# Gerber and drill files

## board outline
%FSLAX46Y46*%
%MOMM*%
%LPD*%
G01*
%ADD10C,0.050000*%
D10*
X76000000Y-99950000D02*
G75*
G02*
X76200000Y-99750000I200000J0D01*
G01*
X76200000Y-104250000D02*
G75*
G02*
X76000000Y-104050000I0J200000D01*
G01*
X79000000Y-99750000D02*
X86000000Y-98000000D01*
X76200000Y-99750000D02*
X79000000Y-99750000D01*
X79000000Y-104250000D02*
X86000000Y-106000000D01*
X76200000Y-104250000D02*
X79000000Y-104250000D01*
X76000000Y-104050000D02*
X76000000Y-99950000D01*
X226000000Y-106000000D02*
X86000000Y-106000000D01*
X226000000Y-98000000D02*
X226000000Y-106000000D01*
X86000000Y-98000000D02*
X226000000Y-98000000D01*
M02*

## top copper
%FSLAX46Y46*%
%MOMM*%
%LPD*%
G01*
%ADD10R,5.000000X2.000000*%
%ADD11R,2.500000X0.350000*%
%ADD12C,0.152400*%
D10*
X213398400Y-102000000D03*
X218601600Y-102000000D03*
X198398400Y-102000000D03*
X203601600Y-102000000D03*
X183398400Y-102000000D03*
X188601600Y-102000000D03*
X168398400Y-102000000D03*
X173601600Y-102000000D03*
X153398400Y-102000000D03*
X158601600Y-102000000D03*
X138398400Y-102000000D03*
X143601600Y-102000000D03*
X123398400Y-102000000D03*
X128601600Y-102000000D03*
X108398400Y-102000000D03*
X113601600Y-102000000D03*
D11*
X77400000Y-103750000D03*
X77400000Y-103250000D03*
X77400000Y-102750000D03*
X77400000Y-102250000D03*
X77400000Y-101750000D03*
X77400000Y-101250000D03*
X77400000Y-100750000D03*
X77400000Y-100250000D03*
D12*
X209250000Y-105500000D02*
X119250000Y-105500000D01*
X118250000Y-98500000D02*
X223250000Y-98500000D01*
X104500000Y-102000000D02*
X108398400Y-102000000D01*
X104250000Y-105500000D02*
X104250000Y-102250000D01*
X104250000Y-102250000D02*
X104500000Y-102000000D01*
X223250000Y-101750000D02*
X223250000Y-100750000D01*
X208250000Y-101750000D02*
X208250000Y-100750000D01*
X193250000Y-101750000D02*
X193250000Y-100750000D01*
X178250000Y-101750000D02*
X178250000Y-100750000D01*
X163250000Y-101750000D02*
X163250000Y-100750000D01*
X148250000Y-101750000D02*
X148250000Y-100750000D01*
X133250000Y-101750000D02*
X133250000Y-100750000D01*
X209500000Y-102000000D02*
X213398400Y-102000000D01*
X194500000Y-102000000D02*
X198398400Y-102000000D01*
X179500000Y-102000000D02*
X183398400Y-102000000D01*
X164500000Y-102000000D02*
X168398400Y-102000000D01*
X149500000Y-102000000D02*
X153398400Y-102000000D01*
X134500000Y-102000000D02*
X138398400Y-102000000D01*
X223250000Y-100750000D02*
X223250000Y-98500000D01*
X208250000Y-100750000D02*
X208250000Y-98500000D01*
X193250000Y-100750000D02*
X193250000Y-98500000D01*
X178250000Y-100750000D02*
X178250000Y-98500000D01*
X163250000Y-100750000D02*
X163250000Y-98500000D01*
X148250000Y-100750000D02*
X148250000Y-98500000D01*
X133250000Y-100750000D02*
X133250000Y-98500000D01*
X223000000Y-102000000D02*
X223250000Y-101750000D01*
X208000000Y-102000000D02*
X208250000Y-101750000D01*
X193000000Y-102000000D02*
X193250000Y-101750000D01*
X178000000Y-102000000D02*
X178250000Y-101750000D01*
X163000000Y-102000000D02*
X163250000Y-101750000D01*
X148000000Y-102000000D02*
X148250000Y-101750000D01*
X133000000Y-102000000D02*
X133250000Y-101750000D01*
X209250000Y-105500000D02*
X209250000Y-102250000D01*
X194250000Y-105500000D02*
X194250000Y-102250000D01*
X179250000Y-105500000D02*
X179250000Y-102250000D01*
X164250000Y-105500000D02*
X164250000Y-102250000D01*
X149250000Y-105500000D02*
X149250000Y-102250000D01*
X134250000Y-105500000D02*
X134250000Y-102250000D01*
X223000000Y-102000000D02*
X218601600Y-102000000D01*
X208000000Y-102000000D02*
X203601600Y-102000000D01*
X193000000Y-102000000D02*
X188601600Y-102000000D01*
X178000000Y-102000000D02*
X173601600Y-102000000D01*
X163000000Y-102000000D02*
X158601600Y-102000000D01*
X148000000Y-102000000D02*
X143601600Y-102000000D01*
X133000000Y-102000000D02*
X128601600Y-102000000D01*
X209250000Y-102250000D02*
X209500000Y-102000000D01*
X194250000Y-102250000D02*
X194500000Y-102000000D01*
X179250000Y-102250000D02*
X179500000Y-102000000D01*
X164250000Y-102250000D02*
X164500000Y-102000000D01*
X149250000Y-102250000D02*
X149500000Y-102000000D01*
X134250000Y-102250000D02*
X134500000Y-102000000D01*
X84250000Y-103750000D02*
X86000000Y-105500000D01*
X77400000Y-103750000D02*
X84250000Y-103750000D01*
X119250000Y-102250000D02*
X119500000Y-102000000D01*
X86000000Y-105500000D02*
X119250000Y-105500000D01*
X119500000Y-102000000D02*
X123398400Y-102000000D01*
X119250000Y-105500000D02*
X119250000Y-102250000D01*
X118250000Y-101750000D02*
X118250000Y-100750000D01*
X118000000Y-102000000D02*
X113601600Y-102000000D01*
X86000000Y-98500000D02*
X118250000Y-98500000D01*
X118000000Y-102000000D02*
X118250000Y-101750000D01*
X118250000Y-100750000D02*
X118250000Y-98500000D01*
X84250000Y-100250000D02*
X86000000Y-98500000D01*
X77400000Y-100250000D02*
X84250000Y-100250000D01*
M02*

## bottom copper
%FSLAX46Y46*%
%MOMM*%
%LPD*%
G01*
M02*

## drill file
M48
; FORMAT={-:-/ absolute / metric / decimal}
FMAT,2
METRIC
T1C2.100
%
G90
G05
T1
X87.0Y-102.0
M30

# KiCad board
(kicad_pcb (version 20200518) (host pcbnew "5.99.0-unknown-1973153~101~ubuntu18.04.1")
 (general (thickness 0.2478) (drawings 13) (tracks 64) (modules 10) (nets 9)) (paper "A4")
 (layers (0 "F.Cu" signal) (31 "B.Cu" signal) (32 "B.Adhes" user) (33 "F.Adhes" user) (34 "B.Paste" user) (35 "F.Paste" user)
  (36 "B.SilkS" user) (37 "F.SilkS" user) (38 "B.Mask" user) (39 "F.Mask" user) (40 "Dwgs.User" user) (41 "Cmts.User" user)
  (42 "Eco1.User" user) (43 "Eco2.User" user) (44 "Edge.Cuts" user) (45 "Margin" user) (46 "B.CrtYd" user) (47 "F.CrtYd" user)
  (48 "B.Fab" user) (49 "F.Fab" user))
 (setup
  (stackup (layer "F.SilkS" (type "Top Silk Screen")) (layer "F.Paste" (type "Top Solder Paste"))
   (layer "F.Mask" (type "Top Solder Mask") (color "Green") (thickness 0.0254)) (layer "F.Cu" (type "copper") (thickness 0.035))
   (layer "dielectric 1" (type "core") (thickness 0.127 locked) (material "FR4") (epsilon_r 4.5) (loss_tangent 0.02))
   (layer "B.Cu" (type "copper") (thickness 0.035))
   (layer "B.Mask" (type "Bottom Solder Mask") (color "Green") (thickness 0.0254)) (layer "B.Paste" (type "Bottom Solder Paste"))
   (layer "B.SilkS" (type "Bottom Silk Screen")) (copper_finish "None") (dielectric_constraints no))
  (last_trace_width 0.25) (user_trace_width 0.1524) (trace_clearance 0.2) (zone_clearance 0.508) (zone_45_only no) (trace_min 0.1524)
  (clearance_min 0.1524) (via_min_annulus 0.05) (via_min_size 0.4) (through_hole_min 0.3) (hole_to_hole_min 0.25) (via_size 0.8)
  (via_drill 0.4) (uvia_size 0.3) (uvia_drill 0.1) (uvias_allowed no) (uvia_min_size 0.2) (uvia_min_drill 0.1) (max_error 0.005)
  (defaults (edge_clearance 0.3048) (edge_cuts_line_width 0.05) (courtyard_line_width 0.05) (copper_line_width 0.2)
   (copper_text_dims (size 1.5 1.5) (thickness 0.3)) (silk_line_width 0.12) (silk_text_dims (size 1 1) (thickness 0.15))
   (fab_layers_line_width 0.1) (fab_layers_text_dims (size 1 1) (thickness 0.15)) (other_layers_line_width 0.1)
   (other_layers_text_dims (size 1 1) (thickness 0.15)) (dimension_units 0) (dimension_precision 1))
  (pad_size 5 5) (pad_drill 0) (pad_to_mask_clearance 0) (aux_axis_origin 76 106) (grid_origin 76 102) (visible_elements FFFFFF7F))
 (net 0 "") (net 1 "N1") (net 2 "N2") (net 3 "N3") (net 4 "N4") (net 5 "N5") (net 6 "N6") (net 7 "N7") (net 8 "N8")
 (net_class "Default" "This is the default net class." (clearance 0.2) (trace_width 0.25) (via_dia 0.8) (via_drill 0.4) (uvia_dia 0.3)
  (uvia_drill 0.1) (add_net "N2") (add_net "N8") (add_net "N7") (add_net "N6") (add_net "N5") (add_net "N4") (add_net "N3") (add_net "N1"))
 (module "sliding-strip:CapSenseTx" (layer "F.Cu") (at 216 102)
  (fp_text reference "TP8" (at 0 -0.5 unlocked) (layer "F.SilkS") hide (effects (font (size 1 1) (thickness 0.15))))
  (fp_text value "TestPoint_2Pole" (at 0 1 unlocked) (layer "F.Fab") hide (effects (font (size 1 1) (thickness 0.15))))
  (pad "1" smd rect (at -2.6016 0) (size 5 2) (layers "F.Cu") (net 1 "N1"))
  (pad "2" smd rect (at 2.6016 0) (size 5 2) (layers "F.Cu") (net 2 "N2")))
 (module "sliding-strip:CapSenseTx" (layer "F.Cu") (at 201 102)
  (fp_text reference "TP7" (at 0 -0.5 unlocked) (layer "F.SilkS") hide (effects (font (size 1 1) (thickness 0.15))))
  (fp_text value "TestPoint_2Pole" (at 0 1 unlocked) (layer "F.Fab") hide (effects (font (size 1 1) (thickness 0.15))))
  (pad "1" smd rect (at -2.6016 0) (size 5 2) (layers "F.Cu") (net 1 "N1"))
  (pad "2" smd rect (at 2.6016 0) (size 5 2) (layers "F.Cu") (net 2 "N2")))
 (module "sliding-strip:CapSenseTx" (layer "F.Cu") (at 186 102)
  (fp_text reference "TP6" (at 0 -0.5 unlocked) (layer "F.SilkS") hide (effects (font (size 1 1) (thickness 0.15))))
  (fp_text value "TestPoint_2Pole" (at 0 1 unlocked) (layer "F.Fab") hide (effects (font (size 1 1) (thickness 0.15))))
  (pad "1" smd rect (at -2.6016 0) (size 5 2) (layers "F.Cu") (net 1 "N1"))
  (pad "2" smd rect (at 2.6016 0) (size 5 2) (layers "F.Cu") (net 2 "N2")))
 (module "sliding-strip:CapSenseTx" (layer "F.Cu") (at 171 102)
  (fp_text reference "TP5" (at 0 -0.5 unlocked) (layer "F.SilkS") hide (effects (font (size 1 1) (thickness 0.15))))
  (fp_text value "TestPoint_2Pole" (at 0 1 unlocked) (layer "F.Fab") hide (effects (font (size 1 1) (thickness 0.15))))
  (pad "1" smd rect (at -2.6016 0) (size 5 2) (layers "F.Cu") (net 1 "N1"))
  (pad "2" smd rect (at 2.6016 0) (size 5 2) (layers "F.Cu") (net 2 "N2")))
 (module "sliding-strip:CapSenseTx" (layer "F.Cu") (at 156 102)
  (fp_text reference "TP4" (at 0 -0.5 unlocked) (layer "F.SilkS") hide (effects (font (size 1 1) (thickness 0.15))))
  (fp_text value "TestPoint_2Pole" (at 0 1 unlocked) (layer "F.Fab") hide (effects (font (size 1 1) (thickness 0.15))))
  (pad "1" smd rect (at -2.6016 0) (size 5 2) (layers "F.Cu") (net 1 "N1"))
  (pad "2" smd rect (at 2.6016 0) (size 5 2) (layers "F.Cu") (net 2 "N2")))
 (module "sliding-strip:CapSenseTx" (layer "F.Cu") (at 141 102)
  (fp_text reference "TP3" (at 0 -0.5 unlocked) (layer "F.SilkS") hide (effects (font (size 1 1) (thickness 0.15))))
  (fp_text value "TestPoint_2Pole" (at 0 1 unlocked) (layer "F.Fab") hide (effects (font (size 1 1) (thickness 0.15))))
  (pad "1" smd rect (at -2.6016 0) (size 5 2) (layers "F.Cu") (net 1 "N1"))
  (pad "2" smd rect (at 2.6016 0) (size 5 2) (layers "F.Cu") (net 2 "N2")))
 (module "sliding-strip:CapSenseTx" (layer "F.Cu") (at 126 102)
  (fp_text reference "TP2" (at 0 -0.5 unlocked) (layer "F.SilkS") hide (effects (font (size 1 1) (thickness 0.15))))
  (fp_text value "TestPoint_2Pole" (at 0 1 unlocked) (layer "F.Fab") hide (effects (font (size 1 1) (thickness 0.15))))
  (pad "1" smd rect (at -2.6016 0) (size 5 2) (layers "F.Cu") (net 1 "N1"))
  (pad "2" smd rect (at 2.6016 0) (size 5 2) (layers "F.Cu") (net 2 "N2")))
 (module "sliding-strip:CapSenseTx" (layer "F.Cu") (at 111 102)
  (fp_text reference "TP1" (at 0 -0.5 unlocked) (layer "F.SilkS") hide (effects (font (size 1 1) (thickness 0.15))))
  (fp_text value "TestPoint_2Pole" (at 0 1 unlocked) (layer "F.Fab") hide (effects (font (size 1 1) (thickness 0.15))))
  (pad "1" smd rect (at -2.6016 0) (size 5 2) (layers "F.Cu") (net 1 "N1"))
  (pad "2" smd rect (at 2.6016 0) (size 5 2) (layers "F.Cu") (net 2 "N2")))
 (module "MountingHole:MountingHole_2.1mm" (layer "F.Cu") (at 87 102)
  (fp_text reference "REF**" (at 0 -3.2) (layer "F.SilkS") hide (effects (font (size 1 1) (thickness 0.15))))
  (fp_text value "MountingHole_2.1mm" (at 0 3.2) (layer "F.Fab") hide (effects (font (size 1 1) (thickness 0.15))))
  (pad "" np_thru_hole circle (at 0 0) (size 2.1 2.1) (drill 2.1) (layers *.Cu *.Mask)))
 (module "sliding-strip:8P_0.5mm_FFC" (layer "F.Cu") (at 77.4 102 -90)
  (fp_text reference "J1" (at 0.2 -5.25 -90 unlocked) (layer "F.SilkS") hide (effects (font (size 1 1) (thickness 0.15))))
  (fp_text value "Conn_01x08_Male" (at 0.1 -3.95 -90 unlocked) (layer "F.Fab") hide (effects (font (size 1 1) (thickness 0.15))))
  (pad "8" smd rect (at 1.75 0 270) (size 0.35 2.5) (layers "F.Cu" "F.Mask") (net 1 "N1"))
  (pad "7" smd rect (at 1.25 0 270) (size 0.35 2.5) (layers "F.Cu" "F.Mask") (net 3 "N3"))
  (pad "6" smd rect (at 0.75 0 270) (size 0.35 2.5) (layers "F.Cu" "F.Mask") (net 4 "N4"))
  (pad "5" smd rect (at 0.25 0 270) (size 0.35 2.5) (layers "F.Cu" "F.Mask") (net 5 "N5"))
  (pad "4" smd rect (at -0.25 0 270) (size 0.35 2.5) (layers "F.Cu" "F.Mask") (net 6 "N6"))
  (pad "3" smd rect (at -0.75 0 270) (size 0.35 2.5) (layers "F.Cu" "F.Mask") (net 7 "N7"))
  (pad "2" smd rect (at -1.25 0 270) (size 0.35 2.5) (layers "F.Cu" "F.Mask") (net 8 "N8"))
  (pad "1" smd rect (at -1.75 0 270) (size 0.35 2.5) (layers "F.Cu" "F.Mask") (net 2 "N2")))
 (gr_arc (start 76.2 99.95) (end 76.2 99.75) (angle -90) (layer "Edge.Cuts") (width 0.05))
 (gr_arc (start 76.2 104.05) (end 76 104.05) (angle -90) (layer "Edge.Cuts") (width 0.05))
 (gr_line (start 79 99.75) (end 86 98) (layer "Edge.Cuts") (width 0.05))
 (gr_line (start 76.2 99.75) (end 79 99.75) (layer "Edge.Cuts") (width 0.05))
 (gr_line (start 79 104.25) (end 86 106) (layer "Edge.Cuts") (width 0.05))
 (gr_line (start 76.2 104.25) (end 79 104.25) (layer "Edge.Cuts") (width 0.05))
 (gr_line (start 76 104.05) (end 76 99.95) (layer "Edge.Cuts") (width 0.05))
 (gr_line (start 226 106) (end 86 106) (layer "Edge.Cuts") (width 0.05))
 (gr_line (start 226 98) (end 226 106) (layer "Edge.Cuts") (width 0.05))
 (gr_line (start 86 98) (end 226 98) (layer "Edge.Cuts") (width 0.05))
 (segment (start 209.25 105.5) (end 119.25 105.5) (width 0.1524) (layer "F.Cu") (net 1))
 (segment (start 118.25 98.5) (end 223.25 98.5) (width 0.1524) (layer "F.Cu") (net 2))
 (segment (start 104.5 102) (end 108.3984 102) (width 0.1524) (layer "F.Cu") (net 1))
 (segment (start 104.25 105.5) (end 104.25 102.25) (width 0.1524) (layer "F.Cu") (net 1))
 (segment (start 104.25 102.25) (end 104.5 102) (width 0.1524) (layer "F.Cu") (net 1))
 (segment (start 223.25 101.75) (end 223.25 100.75) (width 0.1524) (layer "F.Cu") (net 2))
 (segment (start 208.25 101.75) (end 208.25 100.75) (width 0.1524) (layer "F.Cu") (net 2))
 (segment (start 193.25 101.75) (end 193.25 100.75) (width 0.1524) (layer "F.Cu") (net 2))
 (segment (start 178.25 101.75) (end 178.25 100.75) (width 0.1524) (layer "F.Cu") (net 2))
 (segment (start 163.25 101.75) (end 163.25 100.75) (width 0.1524) (layer "F.Cu") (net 2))
 (segment (start 148.25 101.75) (end 148.25 100.75) (width 0.1524) (layer "F.Cu") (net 2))
 (segment (start 133.25 101.75) (end 133.25 100.75) (width 0.1524) (layer "F.Cu") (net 2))
 (segment (start 209.5 102) (end 213.3984 102) (width 0.1524) (layer "F.Cu") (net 1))
 (segment (start 194.5 102) (end 198.3984 102) (width 0.1524) (layer "F.Cu") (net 1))
 (segment (start 179.5 102) (end 183.3984 102) (width 0.1524) (layer "F.Cu") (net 1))
 (segment (start 164.5 102) (end 168.3984 102) (width 0.1524) (layer "F.Cu") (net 1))
 (segment (start 149.5 102) (end 153.3984 102) (width 0.1524) (layer "F.Cu") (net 1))
 (segment (start 134.5 102) (end 138.3984 102) (width 0.1524) (layer "F.Cu") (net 1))
 (segment (start 223.25 100.75) (end 223.25 98.5) (width 0.1524) (layer "F.Cu") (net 2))
 (segment (start 208.25 100.75) (end 208.25 98.5) (width 0.1524) (layer "F.Cu") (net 2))
 (segment (start 193.25 100.75) (end 193.25 98.5) (width 0.1524) (layer "F.Cu") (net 2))
 (segment (start 178.25 100.75) (end 178.25 98.5) (width 0.1524) (layer "F.Cu") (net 2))
 (segment (start 163.25 100.75) (end 163.25 98.5) (width 0.1524) (layer "F.Cu") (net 2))
 (segment (start 148.25 100.75) (end 148.25 98.5) (width 0.1524) (layer "F.Cu") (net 2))
 (segment (start 133.25 100.75) (end 133.25 98.5) (width 0.1524) (layer "F.Cu") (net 2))
 (segment (start 223 102) (end 223.25 101.75) (width 0.1524) (layer "F.Cu") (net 2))
 (segment (start 208 102) (end 208.25 101.75) (width 0.1524) (layer "F.Cu") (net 2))
 (segment (start 193 102) (end 193.25 101.75) (width 0.1524) (layer "F.Cu") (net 2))
 (segment (start 178 102) (end 178.25 101.75) (width 0.1524) (layer "F.Cu") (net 2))
 (segment (start 163 102) (end 163.25 101.75) (width 0.1524) (layer "F.Cu") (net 2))
 (segment (start 148 102) (end 148.25 101.75) (width 0.1524) (layer "F.Cu") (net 2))
 (segment (start 133 102) (end 133.25 101.75) (width 0.1524) (layer "F.Cu") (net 2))
 (segment (start 209.25 105.5) (end 209.25 102.25) (width 0.1524) (layer "F.Cu") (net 1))
 (segment (start 194.25 105.5) (end 194.25 102.25) (width 0.1524) (layer "F.Cu") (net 1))
 (segment (start 179.25 105.5) (end 179.25 102.25) (width 0.1524) (layer "F.Cu") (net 1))
 (segment (start 164.25 105.5) (end 164.25 102.25) (width 0.1524) (layer "F.Cu") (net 1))
 (segment (start 149.25 105.5) (end 149.25 102.25) (width 0.1524) (layer "F.Cu") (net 1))
 (segment (start 134.25 105.5) (end 134.25 102.25) (width 0.1524) (layer "F.Cu") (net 1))
 (segment (start 223 102) (end 218.6016 102) (width 0.1524) (layer "F.Cu") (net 2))
 (segment (start 208 102) (end 203.6016 102) (width 0.1524) (layer "F.Cu") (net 2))
 (segment (start 193 102) (end 188.6016 102) (width 0.1524) (layer "F.Cu") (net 2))
 (segment (start 178 102) (end 173.6016 102) (width 0.1524) (layer "F.Cu") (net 2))
 (segment (start 163 102) (end 158.6016 102) (width 0.1524) (layer "F.Cu") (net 2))
 (segment (start 148 102) (end 143.6016 102) (width 0.1524) (layer "F.Cu") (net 2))
 (segment (start 133 102) (end 128.6016 102) (width 0.1524) (layer "F.Cu") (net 2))
 (segment (start 209.25 102.25) (end 209.5 102) (width 0.1524) (layer "F.Cu") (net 1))
 (segment (start 194.25 102.25) (end 194.5 102) (width 0.1524) (layer "F.Cu") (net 1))
 (segment (start 179.25 102.25) (end 179.5 102) (width 0.1524) (layer "F.Cu") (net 1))
 (segment (start 164.25 102.25) (end 164.5 102) (width 0.1524) (layer "F.Cu") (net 1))
 (segment (start 149.25 102.25) (end 149.5 102) (width 0.1524) (layer "F.Cu") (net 1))
 (segment (start 134.25 102.25) (end 134.5 102) (width 0.1524) (layer "F.Cu") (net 1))
 (segment (start 84.25 103.75) (end 86 105.5) (width 0.1524) (layer "F.Cu") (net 1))
 (segment (start 77.4 103.75) (end 84.25 103.75) (width 0.1524) (layer "F.Cu") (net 1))
 (segment (start 119.25 102.25) (end 119.5 102) (width 0.1524) (layer "F.Cu") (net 1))
 (segment (start 86 105.5) (end 119.25 105.5) (width 0.1524) (layer "F.Cu") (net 1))
 (segment (start 119.5 102) (end 123.3984 102) (width 0.1524) (layer "F.Cu") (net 1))
 (segment (start 119.25 105.5) (end 119.25 102.25) (width 0.1524) (layer "F.Cu") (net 1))
 (segment (start 118.25 101.75) (end 118.25 100.75) (width 0.1524) (layer "F.Cu") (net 2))
 (segment (start 118 102) (end 113.6016 102) (width 0.1524) (layer "F.Cu") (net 2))
 (segment (start 86 98.5) (end 118.25 98.5) (width 0.1524) (layer "F.Cu") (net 2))
 (segment (start 118 102) (end 118.25 101.75) (width 0.1524) (layer "F.Cu") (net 2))
 (segment (start 118.25 100.75) (end 118.25 98.5) (width 0.1524) (layer "F.Cu") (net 2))
 (segment (start 84.25 100.25) (end 86 98.5) (width 0.1524) (layer "F.Cu") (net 2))
 (segment (start 77.4 100.25) (end 84.25 100.25) (width 0.1524) (layer "F.Cu") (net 2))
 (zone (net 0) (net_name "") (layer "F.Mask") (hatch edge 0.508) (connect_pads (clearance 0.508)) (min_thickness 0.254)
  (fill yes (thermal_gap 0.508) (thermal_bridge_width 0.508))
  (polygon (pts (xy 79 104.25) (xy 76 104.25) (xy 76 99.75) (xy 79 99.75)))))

